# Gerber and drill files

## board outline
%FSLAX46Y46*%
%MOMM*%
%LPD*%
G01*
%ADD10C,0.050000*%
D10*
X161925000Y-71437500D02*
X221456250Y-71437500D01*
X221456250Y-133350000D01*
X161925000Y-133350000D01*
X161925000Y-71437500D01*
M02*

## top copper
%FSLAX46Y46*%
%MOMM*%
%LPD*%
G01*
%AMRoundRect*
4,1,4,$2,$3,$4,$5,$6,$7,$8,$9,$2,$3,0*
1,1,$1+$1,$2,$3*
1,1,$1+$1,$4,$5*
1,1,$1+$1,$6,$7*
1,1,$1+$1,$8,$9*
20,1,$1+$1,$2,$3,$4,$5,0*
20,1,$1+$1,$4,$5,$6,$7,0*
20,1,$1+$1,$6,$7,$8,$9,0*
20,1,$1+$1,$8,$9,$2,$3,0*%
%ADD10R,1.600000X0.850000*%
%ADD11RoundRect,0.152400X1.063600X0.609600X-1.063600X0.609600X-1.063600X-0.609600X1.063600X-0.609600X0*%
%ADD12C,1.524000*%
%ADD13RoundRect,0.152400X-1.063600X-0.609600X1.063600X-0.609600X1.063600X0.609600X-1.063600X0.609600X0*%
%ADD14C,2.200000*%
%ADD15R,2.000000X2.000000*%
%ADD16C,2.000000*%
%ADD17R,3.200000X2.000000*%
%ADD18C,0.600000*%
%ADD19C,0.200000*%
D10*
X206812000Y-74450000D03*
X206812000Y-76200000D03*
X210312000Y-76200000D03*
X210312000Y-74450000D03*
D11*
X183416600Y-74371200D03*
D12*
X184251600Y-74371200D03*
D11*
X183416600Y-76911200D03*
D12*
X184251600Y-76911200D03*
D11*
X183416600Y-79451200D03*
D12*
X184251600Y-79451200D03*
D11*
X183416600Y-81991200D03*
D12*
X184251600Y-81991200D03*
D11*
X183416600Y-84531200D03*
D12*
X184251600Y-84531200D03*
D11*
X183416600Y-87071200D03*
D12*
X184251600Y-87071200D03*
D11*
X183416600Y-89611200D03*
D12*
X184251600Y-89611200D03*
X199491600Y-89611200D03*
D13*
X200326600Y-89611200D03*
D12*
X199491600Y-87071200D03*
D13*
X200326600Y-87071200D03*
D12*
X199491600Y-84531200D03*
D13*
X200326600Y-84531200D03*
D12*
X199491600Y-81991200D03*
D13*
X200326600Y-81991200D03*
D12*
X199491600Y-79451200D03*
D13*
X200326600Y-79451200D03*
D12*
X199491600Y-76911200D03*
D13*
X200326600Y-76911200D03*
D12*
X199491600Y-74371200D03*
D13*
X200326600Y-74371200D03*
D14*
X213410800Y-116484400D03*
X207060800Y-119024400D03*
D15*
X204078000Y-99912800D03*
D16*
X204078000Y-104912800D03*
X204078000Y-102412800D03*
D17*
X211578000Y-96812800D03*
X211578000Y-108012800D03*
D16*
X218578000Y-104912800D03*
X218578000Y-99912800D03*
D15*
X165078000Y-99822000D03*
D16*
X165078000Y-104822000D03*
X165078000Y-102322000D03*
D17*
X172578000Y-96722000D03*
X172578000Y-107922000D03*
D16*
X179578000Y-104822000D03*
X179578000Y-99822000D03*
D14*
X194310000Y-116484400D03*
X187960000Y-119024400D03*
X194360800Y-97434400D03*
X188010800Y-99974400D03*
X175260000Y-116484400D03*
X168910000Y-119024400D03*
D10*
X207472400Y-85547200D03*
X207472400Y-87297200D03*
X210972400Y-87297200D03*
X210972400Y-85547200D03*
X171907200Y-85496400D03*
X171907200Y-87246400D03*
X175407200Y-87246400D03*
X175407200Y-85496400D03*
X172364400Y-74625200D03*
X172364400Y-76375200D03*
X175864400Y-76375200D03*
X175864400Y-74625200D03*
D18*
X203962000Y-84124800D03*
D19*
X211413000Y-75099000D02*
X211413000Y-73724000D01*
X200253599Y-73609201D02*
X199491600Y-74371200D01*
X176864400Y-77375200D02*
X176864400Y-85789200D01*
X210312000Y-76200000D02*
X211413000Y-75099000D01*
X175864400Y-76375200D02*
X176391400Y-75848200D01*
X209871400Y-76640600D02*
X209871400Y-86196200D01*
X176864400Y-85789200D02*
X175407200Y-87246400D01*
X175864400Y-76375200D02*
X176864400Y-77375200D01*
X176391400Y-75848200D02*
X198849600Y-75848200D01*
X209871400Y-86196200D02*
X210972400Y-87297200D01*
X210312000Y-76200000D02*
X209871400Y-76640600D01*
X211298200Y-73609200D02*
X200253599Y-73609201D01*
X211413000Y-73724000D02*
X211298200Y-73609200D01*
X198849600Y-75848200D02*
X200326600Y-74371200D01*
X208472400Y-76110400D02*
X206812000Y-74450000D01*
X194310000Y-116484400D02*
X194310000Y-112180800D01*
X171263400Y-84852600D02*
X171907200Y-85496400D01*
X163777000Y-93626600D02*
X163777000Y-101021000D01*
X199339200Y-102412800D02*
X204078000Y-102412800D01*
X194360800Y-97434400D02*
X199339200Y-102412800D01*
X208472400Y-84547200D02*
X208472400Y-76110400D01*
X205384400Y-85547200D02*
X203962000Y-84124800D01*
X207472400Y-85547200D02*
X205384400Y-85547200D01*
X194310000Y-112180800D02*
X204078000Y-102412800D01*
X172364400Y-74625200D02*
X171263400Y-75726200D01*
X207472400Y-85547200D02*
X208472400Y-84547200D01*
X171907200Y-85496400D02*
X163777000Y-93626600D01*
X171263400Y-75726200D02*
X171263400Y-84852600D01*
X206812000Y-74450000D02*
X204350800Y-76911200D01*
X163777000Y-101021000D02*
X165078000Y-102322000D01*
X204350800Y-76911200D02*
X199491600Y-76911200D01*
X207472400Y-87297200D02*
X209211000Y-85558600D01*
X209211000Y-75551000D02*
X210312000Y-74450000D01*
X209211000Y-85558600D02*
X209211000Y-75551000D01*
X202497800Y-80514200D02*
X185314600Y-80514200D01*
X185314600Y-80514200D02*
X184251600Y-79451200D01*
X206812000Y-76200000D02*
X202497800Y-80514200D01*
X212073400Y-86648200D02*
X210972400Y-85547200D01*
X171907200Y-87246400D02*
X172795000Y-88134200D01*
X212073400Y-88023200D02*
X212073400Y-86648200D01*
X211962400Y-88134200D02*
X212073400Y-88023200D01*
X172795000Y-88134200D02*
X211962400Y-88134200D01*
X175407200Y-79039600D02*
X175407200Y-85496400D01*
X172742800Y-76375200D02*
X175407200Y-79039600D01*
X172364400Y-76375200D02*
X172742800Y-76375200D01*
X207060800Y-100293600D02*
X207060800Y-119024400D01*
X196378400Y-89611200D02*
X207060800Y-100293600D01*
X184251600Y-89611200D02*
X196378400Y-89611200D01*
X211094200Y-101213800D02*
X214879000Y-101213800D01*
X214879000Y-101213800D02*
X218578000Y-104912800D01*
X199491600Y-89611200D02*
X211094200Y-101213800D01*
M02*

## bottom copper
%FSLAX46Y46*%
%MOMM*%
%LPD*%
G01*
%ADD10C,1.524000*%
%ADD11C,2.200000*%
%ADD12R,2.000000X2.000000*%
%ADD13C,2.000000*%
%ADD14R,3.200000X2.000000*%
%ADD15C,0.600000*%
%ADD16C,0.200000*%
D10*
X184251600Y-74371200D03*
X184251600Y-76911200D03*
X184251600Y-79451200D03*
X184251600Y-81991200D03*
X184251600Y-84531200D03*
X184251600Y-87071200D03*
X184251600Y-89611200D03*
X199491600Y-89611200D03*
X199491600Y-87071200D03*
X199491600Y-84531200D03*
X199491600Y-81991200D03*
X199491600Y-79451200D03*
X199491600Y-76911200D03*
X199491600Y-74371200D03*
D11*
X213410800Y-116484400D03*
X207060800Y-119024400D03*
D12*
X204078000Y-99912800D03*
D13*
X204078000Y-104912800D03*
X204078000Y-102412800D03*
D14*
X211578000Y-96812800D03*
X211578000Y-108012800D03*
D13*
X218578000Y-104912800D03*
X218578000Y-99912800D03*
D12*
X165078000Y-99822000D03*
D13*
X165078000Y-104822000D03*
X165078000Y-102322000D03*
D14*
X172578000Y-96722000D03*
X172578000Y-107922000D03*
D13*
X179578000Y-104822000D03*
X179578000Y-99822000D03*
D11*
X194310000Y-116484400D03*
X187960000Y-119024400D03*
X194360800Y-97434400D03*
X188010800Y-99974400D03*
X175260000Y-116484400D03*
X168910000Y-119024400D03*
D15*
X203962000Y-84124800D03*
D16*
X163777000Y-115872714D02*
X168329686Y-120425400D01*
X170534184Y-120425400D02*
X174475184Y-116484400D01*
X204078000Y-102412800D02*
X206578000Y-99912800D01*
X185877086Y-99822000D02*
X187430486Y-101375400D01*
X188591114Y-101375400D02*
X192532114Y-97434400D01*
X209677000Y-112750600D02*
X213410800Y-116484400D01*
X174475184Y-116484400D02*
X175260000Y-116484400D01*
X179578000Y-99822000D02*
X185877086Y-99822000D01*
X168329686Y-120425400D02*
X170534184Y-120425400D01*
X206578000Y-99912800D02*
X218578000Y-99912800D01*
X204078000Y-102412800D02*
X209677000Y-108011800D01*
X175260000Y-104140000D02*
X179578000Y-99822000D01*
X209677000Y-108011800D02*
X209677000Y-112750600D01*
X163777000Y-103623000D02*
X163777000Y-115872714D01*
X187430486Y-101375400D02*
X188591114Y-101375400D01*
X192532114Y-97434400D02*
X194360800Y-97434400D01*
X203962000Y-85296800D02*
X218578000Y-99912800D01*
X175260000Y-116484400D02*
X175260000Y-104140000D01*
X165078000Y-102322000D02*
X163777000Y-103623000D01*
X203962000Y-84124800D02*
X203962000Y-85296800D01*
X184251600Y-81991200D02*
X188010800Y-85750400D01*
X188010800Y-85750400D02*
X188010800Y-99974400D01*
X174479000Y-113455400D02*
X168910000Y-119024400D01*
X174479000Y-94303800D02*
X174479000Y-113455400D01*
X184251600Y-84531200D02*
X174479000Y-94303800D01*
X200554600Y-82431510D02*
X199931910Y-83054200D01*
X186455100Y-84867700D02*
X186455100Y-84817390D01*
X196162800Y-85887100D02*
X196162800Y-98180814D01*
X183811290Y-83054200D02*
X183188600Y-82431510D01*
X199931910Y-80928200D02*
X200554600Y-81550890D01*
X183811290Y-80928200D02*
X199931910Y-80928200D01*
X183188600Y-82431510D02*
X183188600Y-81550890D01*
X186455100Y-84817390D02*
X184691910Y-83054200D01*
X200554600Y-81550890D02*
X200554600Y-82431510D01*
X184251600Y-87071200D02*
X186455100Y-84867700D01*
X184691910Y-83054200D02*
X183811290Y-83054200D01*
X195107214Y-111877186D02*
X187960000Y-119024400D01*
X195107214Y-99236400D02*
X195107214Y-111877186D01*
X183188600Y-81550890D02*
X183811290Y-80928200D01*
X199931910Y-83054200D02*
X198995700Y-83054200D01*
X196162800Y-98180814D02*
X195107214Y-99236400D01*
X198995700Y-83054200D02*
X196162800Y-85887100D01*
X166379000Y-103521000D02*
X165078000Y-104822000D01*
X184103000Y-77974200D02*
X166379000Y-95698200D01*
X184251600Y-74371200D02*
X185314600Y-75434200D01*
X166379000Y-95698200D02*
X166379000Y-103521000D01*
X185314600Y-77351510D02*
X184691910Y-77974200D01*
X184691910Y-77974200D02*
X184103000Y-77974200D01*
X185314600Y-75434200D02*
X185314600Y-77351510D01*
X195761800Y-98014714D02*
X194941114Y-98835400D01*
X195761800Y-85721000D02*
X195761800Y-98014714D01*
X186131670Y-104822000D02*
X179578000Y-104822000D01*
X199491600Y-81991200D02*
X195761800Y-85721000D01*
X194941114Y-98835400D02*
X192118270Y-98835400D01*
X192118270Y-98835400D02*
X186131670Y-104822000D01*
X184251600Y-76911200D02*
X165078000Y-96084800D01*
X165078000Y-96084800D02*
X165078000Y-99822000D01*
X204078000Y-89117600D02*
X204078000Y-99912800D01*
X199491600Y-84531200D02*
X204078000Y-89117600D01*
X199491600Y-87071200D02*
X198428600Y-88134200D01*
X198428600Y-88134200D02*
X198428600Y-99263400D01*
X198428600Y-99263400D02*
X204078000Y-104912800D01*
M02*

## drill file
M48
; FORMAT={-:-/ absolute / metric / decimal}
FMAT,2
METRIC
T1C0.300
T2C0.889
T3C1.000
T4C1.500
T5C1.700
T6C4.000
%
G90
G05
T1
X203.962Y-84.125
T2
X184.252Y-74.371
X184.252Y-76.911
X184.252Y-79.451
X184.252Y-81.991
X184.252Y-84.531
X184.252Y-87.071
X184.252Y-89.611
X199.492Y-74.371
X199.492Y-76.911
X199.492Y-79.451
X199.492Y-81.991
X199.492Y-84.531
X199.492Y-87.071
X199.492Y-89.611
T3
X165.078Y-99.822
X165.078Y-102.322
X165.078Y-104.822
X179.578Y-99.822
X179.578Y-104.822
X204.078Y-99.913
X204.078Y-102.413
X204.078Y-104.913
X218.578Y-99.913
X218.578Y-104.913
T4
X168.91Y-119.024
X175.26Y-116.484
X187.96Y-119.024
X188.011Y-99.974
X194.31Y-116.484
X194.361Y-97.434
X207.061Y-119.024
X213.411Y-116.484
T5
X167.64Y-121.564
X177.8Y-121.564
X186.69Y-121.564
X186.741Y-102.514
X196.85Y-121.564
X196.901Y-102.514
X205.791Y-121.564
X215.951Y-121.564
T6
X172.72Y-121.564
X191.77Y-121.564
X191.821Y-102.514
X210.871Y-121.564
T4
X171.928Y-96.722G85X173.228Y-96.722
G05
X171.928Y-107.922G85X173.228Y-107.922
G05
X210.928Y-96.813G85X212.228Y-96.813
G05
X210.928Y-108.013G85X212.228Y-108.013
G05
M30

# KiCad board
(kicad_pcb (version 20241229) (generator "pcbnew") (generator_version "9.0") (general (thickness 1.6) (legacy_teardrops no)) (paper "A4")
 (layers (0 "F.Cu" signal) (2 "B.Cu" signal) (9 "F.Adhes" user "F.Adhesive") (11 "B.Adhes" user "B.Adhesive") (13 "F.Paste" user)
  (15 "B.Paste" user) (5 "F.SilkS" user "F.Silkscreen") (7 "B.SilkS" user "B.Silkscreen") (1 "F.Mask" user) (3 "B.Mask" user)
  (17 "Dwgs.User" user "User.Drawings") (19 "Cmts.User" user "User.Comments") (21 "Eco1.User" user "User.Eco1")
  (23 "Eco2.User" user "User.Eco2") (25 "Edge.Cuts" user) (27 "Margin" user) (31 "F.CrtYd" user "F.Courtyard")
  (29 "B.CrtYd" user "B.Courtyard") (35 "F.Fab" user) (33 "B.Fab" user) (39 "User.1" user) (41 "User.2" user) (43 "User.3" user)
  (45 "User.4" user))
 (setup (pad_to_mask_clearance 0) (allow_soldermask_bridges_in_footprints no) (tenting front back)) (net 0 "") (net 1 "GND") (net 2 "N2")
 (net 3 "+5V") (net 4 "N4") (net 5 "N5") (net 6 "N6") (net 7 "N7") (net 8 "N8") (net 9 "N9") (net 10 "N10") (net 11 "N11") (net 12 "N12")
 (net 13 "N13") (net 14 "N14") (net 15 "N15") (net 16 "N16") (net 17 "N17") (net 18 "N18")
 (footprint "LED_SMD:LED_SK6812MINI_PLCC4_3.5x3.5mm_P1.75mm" (layer "F.Cu") (at 208.562 75.325)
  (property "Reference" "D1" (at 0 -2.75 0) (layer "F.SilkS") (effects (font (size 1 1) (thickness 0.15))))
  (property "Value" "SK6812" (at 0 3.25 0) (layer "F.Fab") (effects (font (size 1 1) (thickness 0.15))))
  (pad "1" smd rect (at -1.75 -0.875) (size 1.6 0.85) (layers "F.Cu" "F.Mask" "F.Paste") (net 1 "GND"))
  (pad "2" smd rect (at -1.75 0.875) (size 1.6 0.85) (layers "F.Cu" "F.Mask" "F.Paste") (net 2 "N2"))
  (pad "3" smd rect (at 1.75 0.875) (size 1.6 0.85) (layers "F.Cu" "F.Mask" "F.Paste") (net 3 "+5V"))
  (pad "4" smd rect (at 1.75 -0.875) (size 1.6 0.85) (layers "F.Cu" "F.Mask" "F.Paste") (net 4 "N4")))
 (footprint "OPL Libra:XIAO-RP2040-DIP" (layer "F.Cu") (at 191.8716 81.9912)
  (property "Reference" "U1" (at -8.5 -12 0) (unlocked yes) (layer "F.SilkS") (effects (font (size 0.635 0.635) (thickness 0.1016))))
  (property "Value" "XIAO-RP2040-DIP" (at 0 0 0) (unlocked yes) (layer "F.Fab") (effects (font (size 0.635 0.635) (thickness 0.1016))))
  (pad "1" smd roundrect (at -8.455 -7.62 180) (size 2.432 1.524) (layers "F.Cu" "F.Mask") (roundrect_rratio 0.1) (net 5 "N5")
   (thermal_bridge_angle 45))
  (pad "1" thru_hole circle (at -7.62 -7.62 180) (size 1.524 1.524) (drill 0.889) (layers "*.Cu" "*.Mask") (remove_unused_layers no)
   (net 5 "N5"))
  (pad "2" smd roundrect (at -8.455 -5.08 180) (size 2.432 1.524) (layers "F.Cu" "F.Mask") (roundrect_rratio 0.1) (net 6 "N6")
   (thermal_bridge_angle 45))
  (pad "2" thru_hole circle (at -7.62 -5.08 180) (size 1.524 1.524) (drill 0.889) (layers "*.Cu" "*.Mask") (remove_unused_layers no)
   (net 6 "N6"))
  (pad "3" smd roundrect (at -8.455 -2.54 180) (size 2.432 1.524) (layers "F.Cu" "F.Mask") (roundrect_rratio 0.1) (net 2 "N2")
   (thermal_bridge_angle 45))
  (pad "3" thru_hole circle (at -7.62 -2.54 180) (size 1.524 1.524) (drill 0.889) (layers "*.Cu" "*.Mask") (remove_unused_layers no)
   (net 2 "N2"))
  (pad "4" smd roundrect (at -8.455 0 180) (size 2.432 1.524) (layers "F.Cu" "F.Mask") (roundrect_rratio 0.1) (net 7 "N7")
   (thermal_bridge_angle 45))
  (pad "4" thru_hole circle (at -7.62 0 180) (size 1.524 1.524) (drill 0.889) (layers "*.Cu" "*.Mask") (remove_unused_layers no)
   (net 7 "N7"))
  (pad "5" smd roundrect (at -8.455 2.54 180) (size 2.432 1.524) (layers "F.Cu" "F.Mask") (roundrect_rratio 0.1) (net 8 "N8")
   (thermal_bridge_angle 45))
  (pad "5" thru_hole circle (at -7.62 2.54 180) (size 1.524 1.524) (drill 0.889) (layers "*.Cu" "*.Mask") (remove_unused_layers no)
   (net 8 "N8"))
  (pad "6" smd roundrect (at -8.455 5.08 180) (size 2.432 1.524) (layers "F.Cu" "F.Mask") (roundrect_rratio 0.1) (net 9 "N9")
   (thermal_bridge_angle 45))
  (pad "6" thru_hole circle (at -7.62 5.08 180) (size 1.524 1.524) (drill 0.889) (layers "*.Cu" "*.Mask") (remove_unused_layers no)
   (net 9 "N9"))
  (pad "7" smd roundrect (at -8.455 7.62 180) (size 2.432 1.524) (layers "F.Cu" "F.Mask") (roundrect_rratio 0.1) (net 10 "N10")
   (thermal_bridge_angle 45))
  (pad "7" thru_hole circle (at -7.62 7.62 180) (size 1.524 1.524) (drill 0.889) (layers "*.Cu" "*.Mask") (remove_unused_layers no)
   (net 10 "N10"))
  (pad "8" thru_hole circle (at 7.62 7.62) (size 1.524 1.524) (drill 0.889) (layers "*.Cu" "*.Mask") (remove_unused_layers no)
   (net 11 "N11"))
  (pad "8" smd roundrect (at 8.455 7.62) (size 2.432 1.524) (layers "F.Cu" "F.Mask") (roundrect_rratio 0.1) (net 11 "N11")
   (thermal_bridge_angle 45))
  (pad "9" thru_hole circle (at 7.62 5.08) (size 1.524 1.524) (drill 0.889) (layers "*.Cu" "*.Mask") (remove_unused_layers no)
   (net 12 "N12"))
  (pad "9" smd roundrect (at 8.455 5.08) (size 2.432 1.524) (layers "F.Cu" "F.Mask") (roundrect_rratio 0.1) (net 12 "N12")
   (thermal_bridge_angle 45))
  (pad "10" thru_hole circle (at 7.62 2.54) (size 1.524 1.524) (drill 0.889) (layers "*.Cu" "*.Mask") (remove_unused_layers no)
   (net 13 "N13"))
  (pad "10" smd roundrect (at 8.455 2.54) (size 2.432 1.524) (layers "F.Cu" "F.Mask") (roundrect_rratio 0.1) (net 13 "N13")
   (thermal_bridge_angle 45))
  (pad "11" thru_hole circle (at 7.62 0) (size 1.524 1.524) (drill 0.889) (layers "*.Cu" "*.Mask") (remove_unused_layers no) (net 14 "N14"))
  (pad "11" smd roundrect (at 8.455 0) (size 2.432 1.524) (layers "F.Cu" "F.Mask") (roundrect_rratio 0.1) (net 14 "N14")
   (thermal_bridge_angle 45))
  (pad "12" thru_hole circle (at 7.62 -2.54) (size 1.524 1.524) (drill 0.889) (layers "*.Cu" "*.Mask") (remove_unused_layers no)
   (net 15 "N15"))
  (pad "12" smd roundrect (at 8.455 -2.54) (size 2.432 1.524) (layers "F.Cu" "F.Mask") (roundrect_rratio 0.1) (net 15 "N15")
   (thermal_bridge_angle 45))
  (pad "13" thru_hole circle (at 7.62 -5.08) (size 1.524 1.524) (drill 0.889) (layers "*.Cu" "*.Mask") (remove_unused_layers no)
   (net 1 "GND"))
  (pad "13" smd roundrect (at 8.455 -5.08) (size 2.432 1.524) (layers "F.Cu" "F.Mask") (roundrect_rratio 0.1) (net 1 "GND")
   (thermal_bridge_angle 45))
  (pad "14" thru_hole circle (at 7.62 -7.62) (size 1.524 1.524) (drill 0.889) (layers "*.Cu" "*.Mask") (remove_unused_layers no)
   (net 3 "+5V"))
  (pad "14" smd roundrect (at 8.455 -7.62) (size 2.432 1.524) (layers "F.Cu" "F.Mask") (roundrect_rratio 0.1) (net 3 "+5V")
   (thermal_bridge_angle 45)))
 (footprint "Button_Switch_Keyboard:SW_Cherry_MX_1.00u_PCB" (layer "F.Cu") (at 213.4108 116.4844)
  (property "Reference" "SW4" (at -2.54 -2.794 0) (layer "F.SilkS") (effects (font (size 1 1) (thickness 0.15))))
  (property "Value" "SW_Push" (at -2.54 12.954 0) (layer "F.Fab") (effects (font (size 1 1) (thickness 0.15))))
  (pad "" np_thru_hole circle (at -7.62 5.08) (size 1.7 1.7) (drill 1.7) (layers "*.Cu" "*.Mask"))
  (pad "" np_thru_hole circle (at -2.54 5.08) (size 4 4) (drill 4) (layers "*.Cu" "*.Mask"))
  (pad "" np_thru_hole circle (at 2.54 5.08) (size 1.7 1.7) (drill 1.7) (layers "*.Cu" "*.Mask"))
  (pad "1" thru_hole circle (at 0 0) (size 2.2 2.2) (drill 1.5) (layers "*.Cu" "*.Mask") (remove_unused_layers no) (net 1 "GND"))
  (pad "2" thru_hole circle (at -6.35 2.54) (size 2.2 2.2) (drill 1.5) (layers "*.Cu" "*.Mask") (remove_unused_layers no) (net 10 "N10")))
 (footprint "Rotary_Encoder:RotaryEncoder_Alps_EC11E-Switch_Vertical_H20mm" (layer "F.Cu") (at 204.078 99.9128)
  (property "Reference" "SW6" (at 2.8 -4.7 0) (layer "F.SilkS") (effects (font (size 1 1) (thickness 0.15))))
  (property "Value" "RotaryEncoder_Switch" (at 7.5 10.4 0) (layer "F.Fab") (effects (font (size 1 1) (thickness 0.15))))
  (pad "A" thru_hole rect (at 0 0) (size 2 2) (drill 1) (layers "*.Cu" "*.Mask") (remove_unused_layers no) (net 13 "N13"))
  (pad "B" thru_hole circle (at 0 5) (size 2 2) (drill 1) (layers "*.Cu" "*.Mask") (remove_unused_layers no) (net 12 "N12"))
  (pad "C" thru_hole circle (at 0 2.5) (size 2 2) (drill 1) (layers "*.Cu" "*.Mask") (remove_unused_layers no) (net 1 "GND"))
  (pad "MP" thru_hole rect (at 7.5 -3.1) (size 3.2 2) (drill oval 2.8 1.5) (layers "*.Cu" "*.Mask") (remove_unused_layers no))
  (pad "MP" thru_hole rect (at 7.5 8.1) (size 3.2 2) (drill oval 2.8 1.5) (layers "*.Cu" "*.Mask") (remove_unused_layers no))
  (pad "S1" thru_hole circle (at 14.5 5) (size 2 2) (drill 1) (layers "*.Cu" "*.Mask") (remove_unused_layers no) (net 11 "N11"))
  (pad "S2" thru_hole circle (at 14.5 0) (size 2 2) (drill 1) (layers "*.Cu" "*.Mask") (remove_unused_layers no) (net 1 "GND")))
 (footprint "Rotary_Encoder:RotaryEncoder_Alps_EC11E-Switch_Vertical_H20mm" (layer "F.Cu") (at 165.078 99.822)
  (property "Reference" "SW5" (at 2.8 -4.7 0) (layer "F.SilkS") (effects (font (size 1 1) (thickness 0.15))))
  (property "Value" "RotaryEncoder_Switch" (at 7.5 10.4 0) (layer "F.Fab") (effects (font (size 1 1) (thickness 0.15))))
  (pad "A" thru_hole rect (at 0 0) (size 2 2) (drill 1) (layers "*.Cu" "*.Mask") (remove_unused_layers no) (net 6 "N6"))
  (pad "B" thru_hole circle (at 0 5) (size 2 2) (drill 1) (layers "*.Cu" "*.Mask") (remove_unused_layers no) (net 5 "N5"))
  (pad "C" thru_hole circle (at 0 2.5) (size 2 2) (drill 1) (layers "*.Cu" "*.Mask") (remove_unused_layers no) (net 1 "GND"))
  (pad "MP" thru_hole rect (at 7.5 -3.1) (size 3.2 2) (drill oval 2.8 1.5) (layers "*.Cu" "*.Mask") (remove_unused_layers no))
  (pad "MP" thru_hole rect (at 7.5 8.1) (size 3.2 2) (drill oval 2.8 1.5) (layers "*.Cu" "*.Mask") (remove_unused_layers no))
  (pad "S1" thru_hole circle (at 14.5 5) (size 2 2) (drill 1) (layers "*.Cu" "*.Mask") (remove_unused_layers no) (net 14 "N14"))
  (pad "S2" thru_hole circle (at 14.5 0) (size 2 2) (drill 1) (layers "*.Cu" "*.Mask") (remove_unused_layers no) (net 1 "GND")))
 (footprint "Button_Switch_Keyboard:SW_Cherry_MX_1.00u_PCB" (layer "F.Cu") (at 194.31 116.4844)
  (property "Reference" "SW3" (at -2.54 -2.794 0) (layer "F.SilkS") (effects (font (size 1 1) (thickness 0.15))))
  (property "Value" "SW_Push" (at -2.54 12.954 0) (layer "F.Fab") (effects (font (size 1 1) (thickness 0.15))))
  (pad "" np_thru_hole circle (at -7.62 5.08) (size 1.7 1.7) (drill 1.7) (layers "*.Cu" "*.Mask"))
  (pad "" np_thru_hole circle (at -2.54 5.08) (size 4 4) (drill 4) (layers "*.Cu" "*.Mask"))
  (pad "" np_thru_hole circle (at 2.54 5.08) (size 1.7 1.7) (drill 1.7) (layers "*.Cu" "*.Mask"))
  (pad "1" thru_hole circle (at 0 0) (size 2.2 2.2) (drill 1.5) (layers "*.Cu" "*.Mask") (remove_unused_layers no) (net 1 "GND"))
  (pad "2" thru_hole circle (at -6.35 2.54) (size 2.2 2.2) (drill 1.5) (layers "*.Cu" "*.Mask") (remove_unused_layers no) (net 9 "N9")))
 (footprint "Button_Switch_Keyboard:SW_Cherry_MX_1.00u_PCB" (layer "F.Cu") (at 194.3608 97.4344)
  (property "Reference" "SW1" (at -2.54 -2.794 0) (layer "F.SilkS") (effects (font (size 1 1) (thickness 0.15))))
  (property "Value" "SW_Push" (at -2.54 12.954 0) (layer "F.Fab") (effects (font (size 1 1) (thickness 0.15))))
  (pad "" np_thru_hole circle (at -7.62 5.08) (size 1.7 1.7) (drill 1.7) (layers "*.Cu" "*.Mask"))
  (pad "" np_thru_hole circle (at -2.54 5.08) (size 4 4) (drill 4) (layers "*.Cu" "*.Mask"))
  (pad "" np_thru_hole circle (at 2.54 5.08) (size 1.7 1.7) (drill 1.7) (layers "*.Cu" "*.Mask"))
  (pad "1" thru_hole circle (at 0 0) (size 2.2 2.2) (drill 1.5) (layers "*.Cu" "*.Mask") (remove_unused_layers no) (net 1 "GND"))
  (pad "2" thru_hole circle (at -6.35 2.54) (size 2.2 2.2) (drill 1.5) (layers "*.Cu" "*.Mask") (remove_unused_layers no) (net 7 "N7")))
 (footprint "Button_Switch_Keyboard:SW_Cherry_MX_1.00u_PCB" (layer "F.Cu") (at 175.26 116.4844)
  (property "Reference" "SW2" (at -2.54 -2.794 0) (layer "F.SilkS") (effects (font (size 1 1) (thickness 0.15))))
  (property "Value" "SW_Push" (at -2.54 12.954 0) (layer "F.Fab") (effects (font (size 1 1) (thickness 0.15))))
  (pad "" np_thru_hole circle (at -7.62 5.08) (size 1.7 1.7) (drill 1.7) (layers "*.Cu" "*.Mask"))
  (pad "" np_thru_hole circle (at -2.54 5.08) (size 4 4) (drill 4) (layers "*.Cu" "*.Mask"))
  (pad "" np_thru_hole circle (at 2.54 5.08) (size 1.7 1.7) (drill 1.7) (layers "*.Cu" "*.Mask"))
  (pad "1" thru_hole circle (at 0 0) (size 2.2 2.2) (drill 1.5) (layers "*.Cu" "*.Mask") (remove_unused_layers no) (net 1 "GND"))
  (pad "2" thru_hole circle (at -6.35 2.54) (size 2.2 2.2) (drill 1.5) (layers "*.Cu" "*.Mask") (remove_unused_layers no) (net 8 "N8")))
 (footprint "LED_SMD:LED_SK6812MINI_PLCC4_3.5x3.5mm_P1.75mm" (layer "F.Cu") (at 209.2224 86.4222)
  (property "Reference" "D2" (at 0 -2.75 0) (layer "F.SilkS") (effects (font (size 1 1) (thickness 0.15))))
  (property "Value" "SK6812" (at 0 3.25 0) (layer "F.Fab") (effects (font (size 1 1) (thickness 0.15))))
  (pad "1" smd rect (at -1.75 -0.875) (size 1.6 0.85) (layers "F.Cu" "F.Mask" "F.Paste") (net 1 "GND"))
  (pad "2" smd rect (at -1.75 0.875) (size 1.6 0.85) (layers "F.Cu" "F.Mask" "F.Paste") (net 4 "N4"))
  (pad "3" smd rect (at 1.75 0.875) (size 1.6 0.85) (layers "F.Cu" "F.Mask" "F.Paste") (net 3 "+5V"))
  (pad "4" smd rect (at 1.75 -0.875) (size 1.6 0.85) (layers "F.Cu" "F.Mask" "F.Paste") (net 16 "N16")))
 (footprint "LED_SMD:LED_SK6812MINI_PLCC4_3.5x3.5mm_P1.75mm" (layer "F.Cu") (at 173.6572 86.3714)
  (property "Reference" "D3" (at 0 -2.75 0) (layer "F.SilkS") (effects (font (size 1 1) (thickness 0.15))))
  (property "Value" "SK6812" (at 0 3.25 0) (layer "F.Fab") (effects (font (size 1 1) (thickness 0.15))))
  (pad "1" smd rect (at -1.75 -0.875) (size 1.6 0.85) (layers "F.Cu" "F.Mask" "F.Paste") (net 1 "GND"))
  (pad "2" smd rect (at -1.75 0.875) (size 1.6 0.85) (layers "F.Cu" "F.Mask" "F.Paste") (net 16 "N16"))
  (pad "3" smd rect (at 1.75 0.875) (size 1.6 0.85) (layers "F.Cu" "F.Mask" "F.Paste") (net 3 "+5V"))
  (pad "4" smd rect (at 1.75 -0.875) (size 1.6 0.85) (layers "F.Cu" "F.Mask" "F.Paste") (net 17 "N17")))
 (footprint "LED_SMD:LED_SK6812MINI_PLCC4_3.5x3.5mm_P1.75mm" (layer "F.Cu") (at 174.1144 75.5002)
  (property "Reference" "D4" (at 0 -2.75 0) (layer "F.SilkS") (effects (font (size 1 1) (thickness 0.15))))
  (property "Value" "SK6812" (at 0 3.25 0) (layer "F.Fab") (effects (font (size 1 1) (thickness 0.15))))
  (pad "1" smd rect (at -1.75 -0.875) (size 1.6 0.85) (layers "F.Cu" "F.Mask" "F.Paste") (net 1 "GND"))
  (pad "2" smd rect (at -1.75 0.875) (size 1.6 0.85) (layers "F.Cu" "F.Mask" "F.Paste") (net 17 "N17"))
  (pad "3" smd rect (at 1.75 0.875) (size 1.6 0.85) (layers "F.Cu" "F.Mask" "F.Paste") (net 3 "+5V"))
  (pad "4" smd rect (at 1.75 -0.875) (size 1.6 0.85) (layers "F.Cu" "F.Mask" "F.Paste") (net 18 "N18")))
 (gr_rect (start 161.925 71.4375) (end 221.45625 133.35) (stroke (width 0.05) (type default)) (fill no) (layer "Edge.Cuts"))
 (segment (start 211.413 75.099) (end 211.413 73.724) (width 0.2) (layer "F.Cu") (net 3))
 (segment (start 200.253599 73.609201) (end 199.4916 74.3712) (width 0.2) (layer "F.Cu") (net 3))
 (segment (start 176.8644 77.3752) (end 176.8644 85.7892) (width 0.2) (layer "F.Cu") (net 3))
 (segment (start 210.312 76.2) (end 211.413 75.099) (width 0.2) (layer "F.Cu") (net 3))
 (segment (start 175.8644 76.3752) (end 176.3914 75.8482) (width 0.2) (layer "F.Cu") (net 3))
 (segment (start 209.8714 76.6406) (end 209.8714 86.1962) (width 0.2) (layer "F.Cu") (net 3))
 (segment (start 176.8644 85.7892) (end 175.4072 87.2464) (width 0.2) (layer "F.Cu") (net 3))
 (segment (start 175.8644 76.3752) (end 176.8644 77.3752) (width 0.2) (layer "F.Cu") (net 3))
 (segment (start 176.3914 75.8482) (end 198.8496 75.8482) (width 0.2) (layer "F.Cu") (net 3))
 (segment (start 209.8714 86.1962) (end 210.9724 87.2972) (width 0.2) (layer "F.Cu") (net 3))
 (segment (start 210.312 76.2) (end 209.8714 76.6406) (width 0.2) (layer "F.Cu") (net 3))
 (segment (start 211.2982 73.6092) (end 200.253599 73.609201) (width 0.2) (layer "F.Cu") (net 3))
 (segment (start 211.413 73.724) (end 211.2982 73.6092) (width 0.2) (layer "F.Cu") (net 3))
 (segment (start 198.8496 75.8482) (end 200.3266 74.3712) (width 0.2) (layer "F.Cu") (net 3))
 (segment (start 208.4724 76.1104) (end 206.812 74.45) (width 0.2) (layer "F.Cu") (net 1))
 (segment (start 194.31 116.4844) (end 194.31 112.1808) (width 0.2) (layer "F.Cu") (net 1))
 (segment (start 171.2634 84.8526) (end 171.9072 85.4964) (width 0.2) (layer "F.Cu") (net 1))
 (segment (start 163.777 93.6266) (end 163.777 101.021) (width 0.2) (layer "F.Cu") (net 1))
 (segment (start 199.3392 102.4128) (end 204.078 102.4128) (width 0.2) (layer "F.Cu") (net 1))
 (segment (start 194.3608 97.4344) (end 199.3392 102.4128) (width 0.2) (layer "F.Cu") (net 1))
 (segment (start 208.4724 84.5472) (end 208.4724 76.1104) (width 0.2) (layer "F.Cu") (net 1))
 (segment (start 205.3844 85.5472) (end 203.962 84.1248) (width 0.2) (layer "F.Cu") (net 1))
 (segment (start 207.4724 85.5472) (end 205.3844 85.5472) (width 0.2) (layer "F.Cu") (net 1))
 (segment (start 194.31 112.1808) (end 204.078 102.4128) (width 0.2) (layer "F.Cu") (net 1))
 (segment (start 172.3644 74.6252) (end 171.2634 75.7262) (width 0.2) (layer "F.Cu") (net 1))
 (segment (start 207.4724 85.5472) (end 208.4724 84.5472) (width 0.2) (layer "F.Cu") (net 1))
 (segment (start 171.9072 85.4964) (end 163.777 93.6266) (width 0.2) (layer "F.Cu") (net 1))
 (segment (start 171.2634 75.7262) (end 171.2634 84.8526) (width 0.2) (layer "F.Cu") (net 1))
 (segment (start 206.812 74.45) (end 204.3508 76.9112) (width 0.2) (layer "F.Cu") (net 1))
 (segment (start 163.777 101.021) (end 165.078 102.322) (width 0.2) (layer "F.Cu") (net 1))
 (segment (start 204.3508 76.9112) (end 199.4916 76.9112) (width 0.2) (layer "F.Cu") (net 1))
 (via (at 203.962 84.1248) (size 0.6) (drill 0.3) (layers "F.Cu" "B.Cu") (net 1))
 (segment (start 163.777 115.872714) (end 168.329686 120.4254) (width 0.2) (layer "B.Cu") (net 1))
 (segment (start 170.534184 120.4254) (end 174.475184 116.4844) (width 0.2) (layer "B.Cu") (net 1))
 (segment (start 204.078 102.4128) (end 206.578 99.9128) (width 0.2) (layer "B.Cu") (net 1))
 (segment (start 185.877086 99.822) (end 187.430486 101.3754) (width 0.2) (layer "B.Cu") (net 1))
 (segment (start 188.591114 101.3754) (end 192.532114 97.4344) (width 0.2) (layer "B.Cu") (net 1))
 (segment (start 209.677 112.7506) (end 213.4108 116.4844) (width 0.2) (layer "B.Cu") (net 1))
 (segment (start 174.475184 116.4844) (end 175.26 116.4844) (width 0.2) (layer "B.Cu") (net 1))
 (segment (start 179.578 99.822) (end 185.877086 99.822) (width 0.2) (layer "B.Cu") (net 1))
 (segment (start 168.329686 120.4254) (end 170.534184 120.4254) (width 0.2) (layer "B.Cu") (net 1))
 (segment (start 206.578 99.9128) (end 218.578 99.9128) (width 0.2) (layer "B.Cu") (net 1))
 (segment (start 204.078 102.4128) (end 209.677 108.0118) (width 0.2) (layer "B.Cu") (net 1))
 (segment (start 175.26 104.14) (end 179.578 99.822) (width 0.2) (layer "B.Cu") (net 1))
 (segment (start 209.677 108.0118) (end 209.677 112.7506) (width 0.2) (layer "B.Cu") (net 1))
 (segment (start 163.777 103.623) (end 163.777 115.872714) (width 0.2) (layer "B.Cu") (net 1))
 (segment (start 187.430486 101.3754) (end 188.591114 101.3754) (width 0.2) (layer "B.Cu") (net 1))
 (segment (start 192.532114 97.4344) (end 194.3608 97.4344) (width 0.2) (layer "B.Cu") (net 1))
 (segment (start 203.962 85.2968) (end 218.578 99.9128) (width 0.2) (layer "B.Cu") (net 1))
 (segment (start 175.26 116.4844) (end 175.26 104.14) (width 0.2) (layer "B.Cu") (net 1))
 (segment (start 165.078 102.322) (end 163.777 103.623) (width 0.2) (layer "B.Cu") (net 1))
 (segment (start 203.962 84.1248) (end 203.962 85.2968) (width 0.2) (layer "B.Cu") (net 1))
 (segment (start 207.4724 87.2972) (end 209.211 85.5586) (width 0.2) (layer "F.Cu") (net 4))
 (segment (start 209.211 75.551) (end 210.312 74.45) (width 0.2) (layer "F.Cu") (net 4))
 (segment (start 209.211 85.5586) (end 209.211 75.551) (width 0.2) (layer "F.Cu") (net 4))
 (segment (start 202.4978 80.5142) (end 185.3146 80.5142) (width 0.2) (layer "F.Cu") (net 2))
 (segment (start 185.3146 80.5142) (end 184.2516 79.4512) (width 0.2) (layer "F.Cu") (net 2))
 (segment (start 206.812 76.2) (end 202.4978 80.5142) (width 0.2) (layer "F.Cu") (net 2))
 (segment (start 212.0734 86.6482) (end 210.9724 85.5472) (width 0.2) (layer "F.Cu") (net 16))
 (segment (start 171.9072 87.2464) (end 172.795 88.1342) (width 0.2) (layer "F.Cu") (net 16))
 (segment (start 212.0734 88.0232) (end 212.0734 86.6482) (width 0.2) (layer "F.Cu") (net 16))
 (segment (start 211.9624 88.1342) (end 212.0734 88.0232) (width 0.2) (layer "F.Cu") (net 16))
 (segment (start 172.795 88.1342) (end 211.9624 88.1342) (width 0.2) (layer "F.Cu") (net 16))
 (segment (start 175.4072 79.0396) (end 175.4072 85.4964) (width 0.2) (layer "F.Cu") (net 17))
 (segment (start 172.7428 76.3752) (end 175.4072 79.0396) (width 0.2) (layer "F.Cu") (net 17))
 (segment (start 172.3644 76.3752) (end 172.7428 76.3752) (width 0.2) (layer "F.Cu") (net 17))
 (segment (start 184.2516 81.9912) (end 188.0108 85.7504) (width 0.2) (layer "B.Cu") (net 7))
 (segment (start 188.0108 85.7504) (end 188.0108 99.9744) (width 0.2) (layer "B.Cu") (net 7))
 (segment (start 174.479 113.4554) (end 168.91 119.0244) (width 0.2) (layer "B.Cu") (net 8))
 (segment (start 174.479 94.3038) (end 174.479 113.4554) (width 0.2) (layer "B.Cu") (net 8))
 (segment (start 184.2516 84.5312) (end 174.479 94.3038) (width 0.2) (layer "B.Cu") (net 8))
 (segment (start 200.5546 82.43151) (end 199.93191 83.0542) (width 0.2) (layer "B.Cu") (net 9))
 (segment (start 186.4551 84.8677) (end 186.4551 84.81739) (width 0.2) (layer "B.Cu") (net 9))
 (segment (start 196.1628 85.8871) (end 196.1628 98.180814) (width 0.2) (layer "B.Cu") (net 9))
 (segment (start 183.81129 83.0542) (end 183.1886 82.43151) (width 0.2) (layer "B.Cu") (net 9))
 (segment (start 199.93191 80.9282) (end 200.5546 81.55089) (width 0.2) (layer "B.Cu") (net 9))
 (segment (start 183.81129 80.9282) (end 199.93191 80.9282) (width 0.2) (layer "B.Cu") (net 9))
 (segment (start 183.1886 82.43151) (end 183.1886 81.55089) (width 0.2) (layer "B.Cu") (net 9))
 (segment (start 186.4551 84.81739) (end 184.69191 83.0542) (width 0.2) (layer "B.Cu") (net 9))
 (segment (start 200.5546 81.55089) (end 200.5546 82.43151) (width 0.2) (layer "B.Cu") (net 9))
 (segment (start 184.2516 87.0712) (end 186.4551 84.8677) (width 0.2) (layer "B.Cu") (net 9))
 (segment (start 184.69191 83.0542) (end 183.81129 83.0542) (width 0.2) (layer "B.Cu") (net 9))
 (segment (start 195.107214 111.877186) (end 187.96 119.0244) (width 0.2) (layer "B.Cu") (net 9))
 (segment (start 195.107214 99.2364) (end 195.107214 111.877186) (width 0.2) (layer "B.Cu") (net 9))
 (segment (start 183.1886 81.55089) (end 183.81129 80.9282) (width 0.2) (layer "B.Cu") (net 9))
 (segment (start 199.93191 83.0542) (end 198.9957 83.0542) (width 0.2) (layer "B.Cu") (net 9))
 (segment (start 196.1628 98.180814) (end 195.107214 99.2364) (width 0.2) (layer "B.Cu") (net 9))
 (segment (start 198.9957 83.0542) (end 196.1628 85.8871) (width 0.2) (layer "B.Cu") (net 9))
 (segment (start 207.0608 100.2936) (end 207.0608 119.0244) (width 0.2) (layer "F.Cu") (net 10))
 (segment (start 196.3784 89.6112) (end 207.0608 100.2936) (width 0.2) (layer "F.Cu") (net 10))
 (segment (start 184.2516 89.6112) (end 196.3784 89.6112) (width 0.2) (layer "F.Cu") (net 10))
 (segment (start 166.379 103.521) (end 165.078 104.822) (width 0.2) (layer "B.Cu") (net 5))
 (segment (start 184.103 77.9742) (end 166.379 95.6982) (width 0.2) (layer "B.Cu") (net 5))
 (segment (start 184.2516 74.3712) (end 185.3146 75.4342) (width 0.2) (layer "B.Cu") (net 5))
 (segment (start 166.379 95.6982) (end 166.379 103.521) (width 0.2) (layer "B.Cu") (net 5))
 (segment (start 185.3146 77.35151) (end 184.69191 77.9742) (width 0.2) (layer "B.Cu") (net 5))
 (segment (start 184.69191 77.9742) (end 184.103 77.9742) (width 0.2) (layer "B.Cu") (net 5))
 (segment (start 185.3146 75.4342) (end 185.3146 77.35151) (width 0.2) (layer "B.Cu") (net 5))
 (segment (start 195.7618 98.014714) (end 194.941114 98.8354) (width 0.2) (layer "B.Cu") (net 14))
 (segment (start 195.7618 85.721) (end 195.7618 98.014714) (width 0.2) (layer "B.Cu") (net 14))
 (segment (start 186.13167 104.822) (end 179.578 104.822) (width 0.2) (layer "B.Cu") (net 14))
 (segment (start 199.4916 81.9912) (end 195.7618 85.721) (width 0.2) (layer "B.Cu") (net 14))
 (segment (start 194.941114 98.8354) (end 192.11827 98.8354) (width 0.2) (layer "B.Cu") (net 14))
 (segment (start 192.11827 98.8354) (end 186.13167 104.822) (width 0.2) (layer "B.Cu") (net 14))
 (segment (start 184.2516 76.9112) (end 165.078 96.0848) (width 0.2) (layer "B.Cu") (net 6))
 (segment (start 165.078 96.0848) (end 165.078 99.822) (width 0.2) (layer "B.Cu") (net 6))
 (segment (start 204.078 89.1176) (end 204.078 99.9128) (width 0.2) (layer "B.Cu") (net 13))
 (segment (start 199.4916 84.5312) (end 204.078 89.1176) (width 0.2) (layer "B.Cu") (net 13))
 (segment (start 211.0942 101.2138) (end 214.879 101.2138) (width 0.2) (layer "F.Cu") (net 11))
 (segment (start 214.879 101.2138) (end 218.578 104.9128) (width 0.2) (layer "F.Cu") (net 11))
 (segment (start 199.4916 89.6112) (end 211.0942 101.2138) (width 0.2) (layer "F.Cu") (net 11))
 (segment (start 199.4916 87.0712) (end 198.4286 88.1342) (width 0.2) (layer "B.Cu") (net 12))
 (segment (start 198.4286 88.1342) (end 198.4286 99.2634) (width 0.2) (layer "B.Cu") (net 12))
 (segment (start 198.4286 99.2634) (end 204.078 104.9128) (width 0.2) (layer "B.Cu") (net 12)))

